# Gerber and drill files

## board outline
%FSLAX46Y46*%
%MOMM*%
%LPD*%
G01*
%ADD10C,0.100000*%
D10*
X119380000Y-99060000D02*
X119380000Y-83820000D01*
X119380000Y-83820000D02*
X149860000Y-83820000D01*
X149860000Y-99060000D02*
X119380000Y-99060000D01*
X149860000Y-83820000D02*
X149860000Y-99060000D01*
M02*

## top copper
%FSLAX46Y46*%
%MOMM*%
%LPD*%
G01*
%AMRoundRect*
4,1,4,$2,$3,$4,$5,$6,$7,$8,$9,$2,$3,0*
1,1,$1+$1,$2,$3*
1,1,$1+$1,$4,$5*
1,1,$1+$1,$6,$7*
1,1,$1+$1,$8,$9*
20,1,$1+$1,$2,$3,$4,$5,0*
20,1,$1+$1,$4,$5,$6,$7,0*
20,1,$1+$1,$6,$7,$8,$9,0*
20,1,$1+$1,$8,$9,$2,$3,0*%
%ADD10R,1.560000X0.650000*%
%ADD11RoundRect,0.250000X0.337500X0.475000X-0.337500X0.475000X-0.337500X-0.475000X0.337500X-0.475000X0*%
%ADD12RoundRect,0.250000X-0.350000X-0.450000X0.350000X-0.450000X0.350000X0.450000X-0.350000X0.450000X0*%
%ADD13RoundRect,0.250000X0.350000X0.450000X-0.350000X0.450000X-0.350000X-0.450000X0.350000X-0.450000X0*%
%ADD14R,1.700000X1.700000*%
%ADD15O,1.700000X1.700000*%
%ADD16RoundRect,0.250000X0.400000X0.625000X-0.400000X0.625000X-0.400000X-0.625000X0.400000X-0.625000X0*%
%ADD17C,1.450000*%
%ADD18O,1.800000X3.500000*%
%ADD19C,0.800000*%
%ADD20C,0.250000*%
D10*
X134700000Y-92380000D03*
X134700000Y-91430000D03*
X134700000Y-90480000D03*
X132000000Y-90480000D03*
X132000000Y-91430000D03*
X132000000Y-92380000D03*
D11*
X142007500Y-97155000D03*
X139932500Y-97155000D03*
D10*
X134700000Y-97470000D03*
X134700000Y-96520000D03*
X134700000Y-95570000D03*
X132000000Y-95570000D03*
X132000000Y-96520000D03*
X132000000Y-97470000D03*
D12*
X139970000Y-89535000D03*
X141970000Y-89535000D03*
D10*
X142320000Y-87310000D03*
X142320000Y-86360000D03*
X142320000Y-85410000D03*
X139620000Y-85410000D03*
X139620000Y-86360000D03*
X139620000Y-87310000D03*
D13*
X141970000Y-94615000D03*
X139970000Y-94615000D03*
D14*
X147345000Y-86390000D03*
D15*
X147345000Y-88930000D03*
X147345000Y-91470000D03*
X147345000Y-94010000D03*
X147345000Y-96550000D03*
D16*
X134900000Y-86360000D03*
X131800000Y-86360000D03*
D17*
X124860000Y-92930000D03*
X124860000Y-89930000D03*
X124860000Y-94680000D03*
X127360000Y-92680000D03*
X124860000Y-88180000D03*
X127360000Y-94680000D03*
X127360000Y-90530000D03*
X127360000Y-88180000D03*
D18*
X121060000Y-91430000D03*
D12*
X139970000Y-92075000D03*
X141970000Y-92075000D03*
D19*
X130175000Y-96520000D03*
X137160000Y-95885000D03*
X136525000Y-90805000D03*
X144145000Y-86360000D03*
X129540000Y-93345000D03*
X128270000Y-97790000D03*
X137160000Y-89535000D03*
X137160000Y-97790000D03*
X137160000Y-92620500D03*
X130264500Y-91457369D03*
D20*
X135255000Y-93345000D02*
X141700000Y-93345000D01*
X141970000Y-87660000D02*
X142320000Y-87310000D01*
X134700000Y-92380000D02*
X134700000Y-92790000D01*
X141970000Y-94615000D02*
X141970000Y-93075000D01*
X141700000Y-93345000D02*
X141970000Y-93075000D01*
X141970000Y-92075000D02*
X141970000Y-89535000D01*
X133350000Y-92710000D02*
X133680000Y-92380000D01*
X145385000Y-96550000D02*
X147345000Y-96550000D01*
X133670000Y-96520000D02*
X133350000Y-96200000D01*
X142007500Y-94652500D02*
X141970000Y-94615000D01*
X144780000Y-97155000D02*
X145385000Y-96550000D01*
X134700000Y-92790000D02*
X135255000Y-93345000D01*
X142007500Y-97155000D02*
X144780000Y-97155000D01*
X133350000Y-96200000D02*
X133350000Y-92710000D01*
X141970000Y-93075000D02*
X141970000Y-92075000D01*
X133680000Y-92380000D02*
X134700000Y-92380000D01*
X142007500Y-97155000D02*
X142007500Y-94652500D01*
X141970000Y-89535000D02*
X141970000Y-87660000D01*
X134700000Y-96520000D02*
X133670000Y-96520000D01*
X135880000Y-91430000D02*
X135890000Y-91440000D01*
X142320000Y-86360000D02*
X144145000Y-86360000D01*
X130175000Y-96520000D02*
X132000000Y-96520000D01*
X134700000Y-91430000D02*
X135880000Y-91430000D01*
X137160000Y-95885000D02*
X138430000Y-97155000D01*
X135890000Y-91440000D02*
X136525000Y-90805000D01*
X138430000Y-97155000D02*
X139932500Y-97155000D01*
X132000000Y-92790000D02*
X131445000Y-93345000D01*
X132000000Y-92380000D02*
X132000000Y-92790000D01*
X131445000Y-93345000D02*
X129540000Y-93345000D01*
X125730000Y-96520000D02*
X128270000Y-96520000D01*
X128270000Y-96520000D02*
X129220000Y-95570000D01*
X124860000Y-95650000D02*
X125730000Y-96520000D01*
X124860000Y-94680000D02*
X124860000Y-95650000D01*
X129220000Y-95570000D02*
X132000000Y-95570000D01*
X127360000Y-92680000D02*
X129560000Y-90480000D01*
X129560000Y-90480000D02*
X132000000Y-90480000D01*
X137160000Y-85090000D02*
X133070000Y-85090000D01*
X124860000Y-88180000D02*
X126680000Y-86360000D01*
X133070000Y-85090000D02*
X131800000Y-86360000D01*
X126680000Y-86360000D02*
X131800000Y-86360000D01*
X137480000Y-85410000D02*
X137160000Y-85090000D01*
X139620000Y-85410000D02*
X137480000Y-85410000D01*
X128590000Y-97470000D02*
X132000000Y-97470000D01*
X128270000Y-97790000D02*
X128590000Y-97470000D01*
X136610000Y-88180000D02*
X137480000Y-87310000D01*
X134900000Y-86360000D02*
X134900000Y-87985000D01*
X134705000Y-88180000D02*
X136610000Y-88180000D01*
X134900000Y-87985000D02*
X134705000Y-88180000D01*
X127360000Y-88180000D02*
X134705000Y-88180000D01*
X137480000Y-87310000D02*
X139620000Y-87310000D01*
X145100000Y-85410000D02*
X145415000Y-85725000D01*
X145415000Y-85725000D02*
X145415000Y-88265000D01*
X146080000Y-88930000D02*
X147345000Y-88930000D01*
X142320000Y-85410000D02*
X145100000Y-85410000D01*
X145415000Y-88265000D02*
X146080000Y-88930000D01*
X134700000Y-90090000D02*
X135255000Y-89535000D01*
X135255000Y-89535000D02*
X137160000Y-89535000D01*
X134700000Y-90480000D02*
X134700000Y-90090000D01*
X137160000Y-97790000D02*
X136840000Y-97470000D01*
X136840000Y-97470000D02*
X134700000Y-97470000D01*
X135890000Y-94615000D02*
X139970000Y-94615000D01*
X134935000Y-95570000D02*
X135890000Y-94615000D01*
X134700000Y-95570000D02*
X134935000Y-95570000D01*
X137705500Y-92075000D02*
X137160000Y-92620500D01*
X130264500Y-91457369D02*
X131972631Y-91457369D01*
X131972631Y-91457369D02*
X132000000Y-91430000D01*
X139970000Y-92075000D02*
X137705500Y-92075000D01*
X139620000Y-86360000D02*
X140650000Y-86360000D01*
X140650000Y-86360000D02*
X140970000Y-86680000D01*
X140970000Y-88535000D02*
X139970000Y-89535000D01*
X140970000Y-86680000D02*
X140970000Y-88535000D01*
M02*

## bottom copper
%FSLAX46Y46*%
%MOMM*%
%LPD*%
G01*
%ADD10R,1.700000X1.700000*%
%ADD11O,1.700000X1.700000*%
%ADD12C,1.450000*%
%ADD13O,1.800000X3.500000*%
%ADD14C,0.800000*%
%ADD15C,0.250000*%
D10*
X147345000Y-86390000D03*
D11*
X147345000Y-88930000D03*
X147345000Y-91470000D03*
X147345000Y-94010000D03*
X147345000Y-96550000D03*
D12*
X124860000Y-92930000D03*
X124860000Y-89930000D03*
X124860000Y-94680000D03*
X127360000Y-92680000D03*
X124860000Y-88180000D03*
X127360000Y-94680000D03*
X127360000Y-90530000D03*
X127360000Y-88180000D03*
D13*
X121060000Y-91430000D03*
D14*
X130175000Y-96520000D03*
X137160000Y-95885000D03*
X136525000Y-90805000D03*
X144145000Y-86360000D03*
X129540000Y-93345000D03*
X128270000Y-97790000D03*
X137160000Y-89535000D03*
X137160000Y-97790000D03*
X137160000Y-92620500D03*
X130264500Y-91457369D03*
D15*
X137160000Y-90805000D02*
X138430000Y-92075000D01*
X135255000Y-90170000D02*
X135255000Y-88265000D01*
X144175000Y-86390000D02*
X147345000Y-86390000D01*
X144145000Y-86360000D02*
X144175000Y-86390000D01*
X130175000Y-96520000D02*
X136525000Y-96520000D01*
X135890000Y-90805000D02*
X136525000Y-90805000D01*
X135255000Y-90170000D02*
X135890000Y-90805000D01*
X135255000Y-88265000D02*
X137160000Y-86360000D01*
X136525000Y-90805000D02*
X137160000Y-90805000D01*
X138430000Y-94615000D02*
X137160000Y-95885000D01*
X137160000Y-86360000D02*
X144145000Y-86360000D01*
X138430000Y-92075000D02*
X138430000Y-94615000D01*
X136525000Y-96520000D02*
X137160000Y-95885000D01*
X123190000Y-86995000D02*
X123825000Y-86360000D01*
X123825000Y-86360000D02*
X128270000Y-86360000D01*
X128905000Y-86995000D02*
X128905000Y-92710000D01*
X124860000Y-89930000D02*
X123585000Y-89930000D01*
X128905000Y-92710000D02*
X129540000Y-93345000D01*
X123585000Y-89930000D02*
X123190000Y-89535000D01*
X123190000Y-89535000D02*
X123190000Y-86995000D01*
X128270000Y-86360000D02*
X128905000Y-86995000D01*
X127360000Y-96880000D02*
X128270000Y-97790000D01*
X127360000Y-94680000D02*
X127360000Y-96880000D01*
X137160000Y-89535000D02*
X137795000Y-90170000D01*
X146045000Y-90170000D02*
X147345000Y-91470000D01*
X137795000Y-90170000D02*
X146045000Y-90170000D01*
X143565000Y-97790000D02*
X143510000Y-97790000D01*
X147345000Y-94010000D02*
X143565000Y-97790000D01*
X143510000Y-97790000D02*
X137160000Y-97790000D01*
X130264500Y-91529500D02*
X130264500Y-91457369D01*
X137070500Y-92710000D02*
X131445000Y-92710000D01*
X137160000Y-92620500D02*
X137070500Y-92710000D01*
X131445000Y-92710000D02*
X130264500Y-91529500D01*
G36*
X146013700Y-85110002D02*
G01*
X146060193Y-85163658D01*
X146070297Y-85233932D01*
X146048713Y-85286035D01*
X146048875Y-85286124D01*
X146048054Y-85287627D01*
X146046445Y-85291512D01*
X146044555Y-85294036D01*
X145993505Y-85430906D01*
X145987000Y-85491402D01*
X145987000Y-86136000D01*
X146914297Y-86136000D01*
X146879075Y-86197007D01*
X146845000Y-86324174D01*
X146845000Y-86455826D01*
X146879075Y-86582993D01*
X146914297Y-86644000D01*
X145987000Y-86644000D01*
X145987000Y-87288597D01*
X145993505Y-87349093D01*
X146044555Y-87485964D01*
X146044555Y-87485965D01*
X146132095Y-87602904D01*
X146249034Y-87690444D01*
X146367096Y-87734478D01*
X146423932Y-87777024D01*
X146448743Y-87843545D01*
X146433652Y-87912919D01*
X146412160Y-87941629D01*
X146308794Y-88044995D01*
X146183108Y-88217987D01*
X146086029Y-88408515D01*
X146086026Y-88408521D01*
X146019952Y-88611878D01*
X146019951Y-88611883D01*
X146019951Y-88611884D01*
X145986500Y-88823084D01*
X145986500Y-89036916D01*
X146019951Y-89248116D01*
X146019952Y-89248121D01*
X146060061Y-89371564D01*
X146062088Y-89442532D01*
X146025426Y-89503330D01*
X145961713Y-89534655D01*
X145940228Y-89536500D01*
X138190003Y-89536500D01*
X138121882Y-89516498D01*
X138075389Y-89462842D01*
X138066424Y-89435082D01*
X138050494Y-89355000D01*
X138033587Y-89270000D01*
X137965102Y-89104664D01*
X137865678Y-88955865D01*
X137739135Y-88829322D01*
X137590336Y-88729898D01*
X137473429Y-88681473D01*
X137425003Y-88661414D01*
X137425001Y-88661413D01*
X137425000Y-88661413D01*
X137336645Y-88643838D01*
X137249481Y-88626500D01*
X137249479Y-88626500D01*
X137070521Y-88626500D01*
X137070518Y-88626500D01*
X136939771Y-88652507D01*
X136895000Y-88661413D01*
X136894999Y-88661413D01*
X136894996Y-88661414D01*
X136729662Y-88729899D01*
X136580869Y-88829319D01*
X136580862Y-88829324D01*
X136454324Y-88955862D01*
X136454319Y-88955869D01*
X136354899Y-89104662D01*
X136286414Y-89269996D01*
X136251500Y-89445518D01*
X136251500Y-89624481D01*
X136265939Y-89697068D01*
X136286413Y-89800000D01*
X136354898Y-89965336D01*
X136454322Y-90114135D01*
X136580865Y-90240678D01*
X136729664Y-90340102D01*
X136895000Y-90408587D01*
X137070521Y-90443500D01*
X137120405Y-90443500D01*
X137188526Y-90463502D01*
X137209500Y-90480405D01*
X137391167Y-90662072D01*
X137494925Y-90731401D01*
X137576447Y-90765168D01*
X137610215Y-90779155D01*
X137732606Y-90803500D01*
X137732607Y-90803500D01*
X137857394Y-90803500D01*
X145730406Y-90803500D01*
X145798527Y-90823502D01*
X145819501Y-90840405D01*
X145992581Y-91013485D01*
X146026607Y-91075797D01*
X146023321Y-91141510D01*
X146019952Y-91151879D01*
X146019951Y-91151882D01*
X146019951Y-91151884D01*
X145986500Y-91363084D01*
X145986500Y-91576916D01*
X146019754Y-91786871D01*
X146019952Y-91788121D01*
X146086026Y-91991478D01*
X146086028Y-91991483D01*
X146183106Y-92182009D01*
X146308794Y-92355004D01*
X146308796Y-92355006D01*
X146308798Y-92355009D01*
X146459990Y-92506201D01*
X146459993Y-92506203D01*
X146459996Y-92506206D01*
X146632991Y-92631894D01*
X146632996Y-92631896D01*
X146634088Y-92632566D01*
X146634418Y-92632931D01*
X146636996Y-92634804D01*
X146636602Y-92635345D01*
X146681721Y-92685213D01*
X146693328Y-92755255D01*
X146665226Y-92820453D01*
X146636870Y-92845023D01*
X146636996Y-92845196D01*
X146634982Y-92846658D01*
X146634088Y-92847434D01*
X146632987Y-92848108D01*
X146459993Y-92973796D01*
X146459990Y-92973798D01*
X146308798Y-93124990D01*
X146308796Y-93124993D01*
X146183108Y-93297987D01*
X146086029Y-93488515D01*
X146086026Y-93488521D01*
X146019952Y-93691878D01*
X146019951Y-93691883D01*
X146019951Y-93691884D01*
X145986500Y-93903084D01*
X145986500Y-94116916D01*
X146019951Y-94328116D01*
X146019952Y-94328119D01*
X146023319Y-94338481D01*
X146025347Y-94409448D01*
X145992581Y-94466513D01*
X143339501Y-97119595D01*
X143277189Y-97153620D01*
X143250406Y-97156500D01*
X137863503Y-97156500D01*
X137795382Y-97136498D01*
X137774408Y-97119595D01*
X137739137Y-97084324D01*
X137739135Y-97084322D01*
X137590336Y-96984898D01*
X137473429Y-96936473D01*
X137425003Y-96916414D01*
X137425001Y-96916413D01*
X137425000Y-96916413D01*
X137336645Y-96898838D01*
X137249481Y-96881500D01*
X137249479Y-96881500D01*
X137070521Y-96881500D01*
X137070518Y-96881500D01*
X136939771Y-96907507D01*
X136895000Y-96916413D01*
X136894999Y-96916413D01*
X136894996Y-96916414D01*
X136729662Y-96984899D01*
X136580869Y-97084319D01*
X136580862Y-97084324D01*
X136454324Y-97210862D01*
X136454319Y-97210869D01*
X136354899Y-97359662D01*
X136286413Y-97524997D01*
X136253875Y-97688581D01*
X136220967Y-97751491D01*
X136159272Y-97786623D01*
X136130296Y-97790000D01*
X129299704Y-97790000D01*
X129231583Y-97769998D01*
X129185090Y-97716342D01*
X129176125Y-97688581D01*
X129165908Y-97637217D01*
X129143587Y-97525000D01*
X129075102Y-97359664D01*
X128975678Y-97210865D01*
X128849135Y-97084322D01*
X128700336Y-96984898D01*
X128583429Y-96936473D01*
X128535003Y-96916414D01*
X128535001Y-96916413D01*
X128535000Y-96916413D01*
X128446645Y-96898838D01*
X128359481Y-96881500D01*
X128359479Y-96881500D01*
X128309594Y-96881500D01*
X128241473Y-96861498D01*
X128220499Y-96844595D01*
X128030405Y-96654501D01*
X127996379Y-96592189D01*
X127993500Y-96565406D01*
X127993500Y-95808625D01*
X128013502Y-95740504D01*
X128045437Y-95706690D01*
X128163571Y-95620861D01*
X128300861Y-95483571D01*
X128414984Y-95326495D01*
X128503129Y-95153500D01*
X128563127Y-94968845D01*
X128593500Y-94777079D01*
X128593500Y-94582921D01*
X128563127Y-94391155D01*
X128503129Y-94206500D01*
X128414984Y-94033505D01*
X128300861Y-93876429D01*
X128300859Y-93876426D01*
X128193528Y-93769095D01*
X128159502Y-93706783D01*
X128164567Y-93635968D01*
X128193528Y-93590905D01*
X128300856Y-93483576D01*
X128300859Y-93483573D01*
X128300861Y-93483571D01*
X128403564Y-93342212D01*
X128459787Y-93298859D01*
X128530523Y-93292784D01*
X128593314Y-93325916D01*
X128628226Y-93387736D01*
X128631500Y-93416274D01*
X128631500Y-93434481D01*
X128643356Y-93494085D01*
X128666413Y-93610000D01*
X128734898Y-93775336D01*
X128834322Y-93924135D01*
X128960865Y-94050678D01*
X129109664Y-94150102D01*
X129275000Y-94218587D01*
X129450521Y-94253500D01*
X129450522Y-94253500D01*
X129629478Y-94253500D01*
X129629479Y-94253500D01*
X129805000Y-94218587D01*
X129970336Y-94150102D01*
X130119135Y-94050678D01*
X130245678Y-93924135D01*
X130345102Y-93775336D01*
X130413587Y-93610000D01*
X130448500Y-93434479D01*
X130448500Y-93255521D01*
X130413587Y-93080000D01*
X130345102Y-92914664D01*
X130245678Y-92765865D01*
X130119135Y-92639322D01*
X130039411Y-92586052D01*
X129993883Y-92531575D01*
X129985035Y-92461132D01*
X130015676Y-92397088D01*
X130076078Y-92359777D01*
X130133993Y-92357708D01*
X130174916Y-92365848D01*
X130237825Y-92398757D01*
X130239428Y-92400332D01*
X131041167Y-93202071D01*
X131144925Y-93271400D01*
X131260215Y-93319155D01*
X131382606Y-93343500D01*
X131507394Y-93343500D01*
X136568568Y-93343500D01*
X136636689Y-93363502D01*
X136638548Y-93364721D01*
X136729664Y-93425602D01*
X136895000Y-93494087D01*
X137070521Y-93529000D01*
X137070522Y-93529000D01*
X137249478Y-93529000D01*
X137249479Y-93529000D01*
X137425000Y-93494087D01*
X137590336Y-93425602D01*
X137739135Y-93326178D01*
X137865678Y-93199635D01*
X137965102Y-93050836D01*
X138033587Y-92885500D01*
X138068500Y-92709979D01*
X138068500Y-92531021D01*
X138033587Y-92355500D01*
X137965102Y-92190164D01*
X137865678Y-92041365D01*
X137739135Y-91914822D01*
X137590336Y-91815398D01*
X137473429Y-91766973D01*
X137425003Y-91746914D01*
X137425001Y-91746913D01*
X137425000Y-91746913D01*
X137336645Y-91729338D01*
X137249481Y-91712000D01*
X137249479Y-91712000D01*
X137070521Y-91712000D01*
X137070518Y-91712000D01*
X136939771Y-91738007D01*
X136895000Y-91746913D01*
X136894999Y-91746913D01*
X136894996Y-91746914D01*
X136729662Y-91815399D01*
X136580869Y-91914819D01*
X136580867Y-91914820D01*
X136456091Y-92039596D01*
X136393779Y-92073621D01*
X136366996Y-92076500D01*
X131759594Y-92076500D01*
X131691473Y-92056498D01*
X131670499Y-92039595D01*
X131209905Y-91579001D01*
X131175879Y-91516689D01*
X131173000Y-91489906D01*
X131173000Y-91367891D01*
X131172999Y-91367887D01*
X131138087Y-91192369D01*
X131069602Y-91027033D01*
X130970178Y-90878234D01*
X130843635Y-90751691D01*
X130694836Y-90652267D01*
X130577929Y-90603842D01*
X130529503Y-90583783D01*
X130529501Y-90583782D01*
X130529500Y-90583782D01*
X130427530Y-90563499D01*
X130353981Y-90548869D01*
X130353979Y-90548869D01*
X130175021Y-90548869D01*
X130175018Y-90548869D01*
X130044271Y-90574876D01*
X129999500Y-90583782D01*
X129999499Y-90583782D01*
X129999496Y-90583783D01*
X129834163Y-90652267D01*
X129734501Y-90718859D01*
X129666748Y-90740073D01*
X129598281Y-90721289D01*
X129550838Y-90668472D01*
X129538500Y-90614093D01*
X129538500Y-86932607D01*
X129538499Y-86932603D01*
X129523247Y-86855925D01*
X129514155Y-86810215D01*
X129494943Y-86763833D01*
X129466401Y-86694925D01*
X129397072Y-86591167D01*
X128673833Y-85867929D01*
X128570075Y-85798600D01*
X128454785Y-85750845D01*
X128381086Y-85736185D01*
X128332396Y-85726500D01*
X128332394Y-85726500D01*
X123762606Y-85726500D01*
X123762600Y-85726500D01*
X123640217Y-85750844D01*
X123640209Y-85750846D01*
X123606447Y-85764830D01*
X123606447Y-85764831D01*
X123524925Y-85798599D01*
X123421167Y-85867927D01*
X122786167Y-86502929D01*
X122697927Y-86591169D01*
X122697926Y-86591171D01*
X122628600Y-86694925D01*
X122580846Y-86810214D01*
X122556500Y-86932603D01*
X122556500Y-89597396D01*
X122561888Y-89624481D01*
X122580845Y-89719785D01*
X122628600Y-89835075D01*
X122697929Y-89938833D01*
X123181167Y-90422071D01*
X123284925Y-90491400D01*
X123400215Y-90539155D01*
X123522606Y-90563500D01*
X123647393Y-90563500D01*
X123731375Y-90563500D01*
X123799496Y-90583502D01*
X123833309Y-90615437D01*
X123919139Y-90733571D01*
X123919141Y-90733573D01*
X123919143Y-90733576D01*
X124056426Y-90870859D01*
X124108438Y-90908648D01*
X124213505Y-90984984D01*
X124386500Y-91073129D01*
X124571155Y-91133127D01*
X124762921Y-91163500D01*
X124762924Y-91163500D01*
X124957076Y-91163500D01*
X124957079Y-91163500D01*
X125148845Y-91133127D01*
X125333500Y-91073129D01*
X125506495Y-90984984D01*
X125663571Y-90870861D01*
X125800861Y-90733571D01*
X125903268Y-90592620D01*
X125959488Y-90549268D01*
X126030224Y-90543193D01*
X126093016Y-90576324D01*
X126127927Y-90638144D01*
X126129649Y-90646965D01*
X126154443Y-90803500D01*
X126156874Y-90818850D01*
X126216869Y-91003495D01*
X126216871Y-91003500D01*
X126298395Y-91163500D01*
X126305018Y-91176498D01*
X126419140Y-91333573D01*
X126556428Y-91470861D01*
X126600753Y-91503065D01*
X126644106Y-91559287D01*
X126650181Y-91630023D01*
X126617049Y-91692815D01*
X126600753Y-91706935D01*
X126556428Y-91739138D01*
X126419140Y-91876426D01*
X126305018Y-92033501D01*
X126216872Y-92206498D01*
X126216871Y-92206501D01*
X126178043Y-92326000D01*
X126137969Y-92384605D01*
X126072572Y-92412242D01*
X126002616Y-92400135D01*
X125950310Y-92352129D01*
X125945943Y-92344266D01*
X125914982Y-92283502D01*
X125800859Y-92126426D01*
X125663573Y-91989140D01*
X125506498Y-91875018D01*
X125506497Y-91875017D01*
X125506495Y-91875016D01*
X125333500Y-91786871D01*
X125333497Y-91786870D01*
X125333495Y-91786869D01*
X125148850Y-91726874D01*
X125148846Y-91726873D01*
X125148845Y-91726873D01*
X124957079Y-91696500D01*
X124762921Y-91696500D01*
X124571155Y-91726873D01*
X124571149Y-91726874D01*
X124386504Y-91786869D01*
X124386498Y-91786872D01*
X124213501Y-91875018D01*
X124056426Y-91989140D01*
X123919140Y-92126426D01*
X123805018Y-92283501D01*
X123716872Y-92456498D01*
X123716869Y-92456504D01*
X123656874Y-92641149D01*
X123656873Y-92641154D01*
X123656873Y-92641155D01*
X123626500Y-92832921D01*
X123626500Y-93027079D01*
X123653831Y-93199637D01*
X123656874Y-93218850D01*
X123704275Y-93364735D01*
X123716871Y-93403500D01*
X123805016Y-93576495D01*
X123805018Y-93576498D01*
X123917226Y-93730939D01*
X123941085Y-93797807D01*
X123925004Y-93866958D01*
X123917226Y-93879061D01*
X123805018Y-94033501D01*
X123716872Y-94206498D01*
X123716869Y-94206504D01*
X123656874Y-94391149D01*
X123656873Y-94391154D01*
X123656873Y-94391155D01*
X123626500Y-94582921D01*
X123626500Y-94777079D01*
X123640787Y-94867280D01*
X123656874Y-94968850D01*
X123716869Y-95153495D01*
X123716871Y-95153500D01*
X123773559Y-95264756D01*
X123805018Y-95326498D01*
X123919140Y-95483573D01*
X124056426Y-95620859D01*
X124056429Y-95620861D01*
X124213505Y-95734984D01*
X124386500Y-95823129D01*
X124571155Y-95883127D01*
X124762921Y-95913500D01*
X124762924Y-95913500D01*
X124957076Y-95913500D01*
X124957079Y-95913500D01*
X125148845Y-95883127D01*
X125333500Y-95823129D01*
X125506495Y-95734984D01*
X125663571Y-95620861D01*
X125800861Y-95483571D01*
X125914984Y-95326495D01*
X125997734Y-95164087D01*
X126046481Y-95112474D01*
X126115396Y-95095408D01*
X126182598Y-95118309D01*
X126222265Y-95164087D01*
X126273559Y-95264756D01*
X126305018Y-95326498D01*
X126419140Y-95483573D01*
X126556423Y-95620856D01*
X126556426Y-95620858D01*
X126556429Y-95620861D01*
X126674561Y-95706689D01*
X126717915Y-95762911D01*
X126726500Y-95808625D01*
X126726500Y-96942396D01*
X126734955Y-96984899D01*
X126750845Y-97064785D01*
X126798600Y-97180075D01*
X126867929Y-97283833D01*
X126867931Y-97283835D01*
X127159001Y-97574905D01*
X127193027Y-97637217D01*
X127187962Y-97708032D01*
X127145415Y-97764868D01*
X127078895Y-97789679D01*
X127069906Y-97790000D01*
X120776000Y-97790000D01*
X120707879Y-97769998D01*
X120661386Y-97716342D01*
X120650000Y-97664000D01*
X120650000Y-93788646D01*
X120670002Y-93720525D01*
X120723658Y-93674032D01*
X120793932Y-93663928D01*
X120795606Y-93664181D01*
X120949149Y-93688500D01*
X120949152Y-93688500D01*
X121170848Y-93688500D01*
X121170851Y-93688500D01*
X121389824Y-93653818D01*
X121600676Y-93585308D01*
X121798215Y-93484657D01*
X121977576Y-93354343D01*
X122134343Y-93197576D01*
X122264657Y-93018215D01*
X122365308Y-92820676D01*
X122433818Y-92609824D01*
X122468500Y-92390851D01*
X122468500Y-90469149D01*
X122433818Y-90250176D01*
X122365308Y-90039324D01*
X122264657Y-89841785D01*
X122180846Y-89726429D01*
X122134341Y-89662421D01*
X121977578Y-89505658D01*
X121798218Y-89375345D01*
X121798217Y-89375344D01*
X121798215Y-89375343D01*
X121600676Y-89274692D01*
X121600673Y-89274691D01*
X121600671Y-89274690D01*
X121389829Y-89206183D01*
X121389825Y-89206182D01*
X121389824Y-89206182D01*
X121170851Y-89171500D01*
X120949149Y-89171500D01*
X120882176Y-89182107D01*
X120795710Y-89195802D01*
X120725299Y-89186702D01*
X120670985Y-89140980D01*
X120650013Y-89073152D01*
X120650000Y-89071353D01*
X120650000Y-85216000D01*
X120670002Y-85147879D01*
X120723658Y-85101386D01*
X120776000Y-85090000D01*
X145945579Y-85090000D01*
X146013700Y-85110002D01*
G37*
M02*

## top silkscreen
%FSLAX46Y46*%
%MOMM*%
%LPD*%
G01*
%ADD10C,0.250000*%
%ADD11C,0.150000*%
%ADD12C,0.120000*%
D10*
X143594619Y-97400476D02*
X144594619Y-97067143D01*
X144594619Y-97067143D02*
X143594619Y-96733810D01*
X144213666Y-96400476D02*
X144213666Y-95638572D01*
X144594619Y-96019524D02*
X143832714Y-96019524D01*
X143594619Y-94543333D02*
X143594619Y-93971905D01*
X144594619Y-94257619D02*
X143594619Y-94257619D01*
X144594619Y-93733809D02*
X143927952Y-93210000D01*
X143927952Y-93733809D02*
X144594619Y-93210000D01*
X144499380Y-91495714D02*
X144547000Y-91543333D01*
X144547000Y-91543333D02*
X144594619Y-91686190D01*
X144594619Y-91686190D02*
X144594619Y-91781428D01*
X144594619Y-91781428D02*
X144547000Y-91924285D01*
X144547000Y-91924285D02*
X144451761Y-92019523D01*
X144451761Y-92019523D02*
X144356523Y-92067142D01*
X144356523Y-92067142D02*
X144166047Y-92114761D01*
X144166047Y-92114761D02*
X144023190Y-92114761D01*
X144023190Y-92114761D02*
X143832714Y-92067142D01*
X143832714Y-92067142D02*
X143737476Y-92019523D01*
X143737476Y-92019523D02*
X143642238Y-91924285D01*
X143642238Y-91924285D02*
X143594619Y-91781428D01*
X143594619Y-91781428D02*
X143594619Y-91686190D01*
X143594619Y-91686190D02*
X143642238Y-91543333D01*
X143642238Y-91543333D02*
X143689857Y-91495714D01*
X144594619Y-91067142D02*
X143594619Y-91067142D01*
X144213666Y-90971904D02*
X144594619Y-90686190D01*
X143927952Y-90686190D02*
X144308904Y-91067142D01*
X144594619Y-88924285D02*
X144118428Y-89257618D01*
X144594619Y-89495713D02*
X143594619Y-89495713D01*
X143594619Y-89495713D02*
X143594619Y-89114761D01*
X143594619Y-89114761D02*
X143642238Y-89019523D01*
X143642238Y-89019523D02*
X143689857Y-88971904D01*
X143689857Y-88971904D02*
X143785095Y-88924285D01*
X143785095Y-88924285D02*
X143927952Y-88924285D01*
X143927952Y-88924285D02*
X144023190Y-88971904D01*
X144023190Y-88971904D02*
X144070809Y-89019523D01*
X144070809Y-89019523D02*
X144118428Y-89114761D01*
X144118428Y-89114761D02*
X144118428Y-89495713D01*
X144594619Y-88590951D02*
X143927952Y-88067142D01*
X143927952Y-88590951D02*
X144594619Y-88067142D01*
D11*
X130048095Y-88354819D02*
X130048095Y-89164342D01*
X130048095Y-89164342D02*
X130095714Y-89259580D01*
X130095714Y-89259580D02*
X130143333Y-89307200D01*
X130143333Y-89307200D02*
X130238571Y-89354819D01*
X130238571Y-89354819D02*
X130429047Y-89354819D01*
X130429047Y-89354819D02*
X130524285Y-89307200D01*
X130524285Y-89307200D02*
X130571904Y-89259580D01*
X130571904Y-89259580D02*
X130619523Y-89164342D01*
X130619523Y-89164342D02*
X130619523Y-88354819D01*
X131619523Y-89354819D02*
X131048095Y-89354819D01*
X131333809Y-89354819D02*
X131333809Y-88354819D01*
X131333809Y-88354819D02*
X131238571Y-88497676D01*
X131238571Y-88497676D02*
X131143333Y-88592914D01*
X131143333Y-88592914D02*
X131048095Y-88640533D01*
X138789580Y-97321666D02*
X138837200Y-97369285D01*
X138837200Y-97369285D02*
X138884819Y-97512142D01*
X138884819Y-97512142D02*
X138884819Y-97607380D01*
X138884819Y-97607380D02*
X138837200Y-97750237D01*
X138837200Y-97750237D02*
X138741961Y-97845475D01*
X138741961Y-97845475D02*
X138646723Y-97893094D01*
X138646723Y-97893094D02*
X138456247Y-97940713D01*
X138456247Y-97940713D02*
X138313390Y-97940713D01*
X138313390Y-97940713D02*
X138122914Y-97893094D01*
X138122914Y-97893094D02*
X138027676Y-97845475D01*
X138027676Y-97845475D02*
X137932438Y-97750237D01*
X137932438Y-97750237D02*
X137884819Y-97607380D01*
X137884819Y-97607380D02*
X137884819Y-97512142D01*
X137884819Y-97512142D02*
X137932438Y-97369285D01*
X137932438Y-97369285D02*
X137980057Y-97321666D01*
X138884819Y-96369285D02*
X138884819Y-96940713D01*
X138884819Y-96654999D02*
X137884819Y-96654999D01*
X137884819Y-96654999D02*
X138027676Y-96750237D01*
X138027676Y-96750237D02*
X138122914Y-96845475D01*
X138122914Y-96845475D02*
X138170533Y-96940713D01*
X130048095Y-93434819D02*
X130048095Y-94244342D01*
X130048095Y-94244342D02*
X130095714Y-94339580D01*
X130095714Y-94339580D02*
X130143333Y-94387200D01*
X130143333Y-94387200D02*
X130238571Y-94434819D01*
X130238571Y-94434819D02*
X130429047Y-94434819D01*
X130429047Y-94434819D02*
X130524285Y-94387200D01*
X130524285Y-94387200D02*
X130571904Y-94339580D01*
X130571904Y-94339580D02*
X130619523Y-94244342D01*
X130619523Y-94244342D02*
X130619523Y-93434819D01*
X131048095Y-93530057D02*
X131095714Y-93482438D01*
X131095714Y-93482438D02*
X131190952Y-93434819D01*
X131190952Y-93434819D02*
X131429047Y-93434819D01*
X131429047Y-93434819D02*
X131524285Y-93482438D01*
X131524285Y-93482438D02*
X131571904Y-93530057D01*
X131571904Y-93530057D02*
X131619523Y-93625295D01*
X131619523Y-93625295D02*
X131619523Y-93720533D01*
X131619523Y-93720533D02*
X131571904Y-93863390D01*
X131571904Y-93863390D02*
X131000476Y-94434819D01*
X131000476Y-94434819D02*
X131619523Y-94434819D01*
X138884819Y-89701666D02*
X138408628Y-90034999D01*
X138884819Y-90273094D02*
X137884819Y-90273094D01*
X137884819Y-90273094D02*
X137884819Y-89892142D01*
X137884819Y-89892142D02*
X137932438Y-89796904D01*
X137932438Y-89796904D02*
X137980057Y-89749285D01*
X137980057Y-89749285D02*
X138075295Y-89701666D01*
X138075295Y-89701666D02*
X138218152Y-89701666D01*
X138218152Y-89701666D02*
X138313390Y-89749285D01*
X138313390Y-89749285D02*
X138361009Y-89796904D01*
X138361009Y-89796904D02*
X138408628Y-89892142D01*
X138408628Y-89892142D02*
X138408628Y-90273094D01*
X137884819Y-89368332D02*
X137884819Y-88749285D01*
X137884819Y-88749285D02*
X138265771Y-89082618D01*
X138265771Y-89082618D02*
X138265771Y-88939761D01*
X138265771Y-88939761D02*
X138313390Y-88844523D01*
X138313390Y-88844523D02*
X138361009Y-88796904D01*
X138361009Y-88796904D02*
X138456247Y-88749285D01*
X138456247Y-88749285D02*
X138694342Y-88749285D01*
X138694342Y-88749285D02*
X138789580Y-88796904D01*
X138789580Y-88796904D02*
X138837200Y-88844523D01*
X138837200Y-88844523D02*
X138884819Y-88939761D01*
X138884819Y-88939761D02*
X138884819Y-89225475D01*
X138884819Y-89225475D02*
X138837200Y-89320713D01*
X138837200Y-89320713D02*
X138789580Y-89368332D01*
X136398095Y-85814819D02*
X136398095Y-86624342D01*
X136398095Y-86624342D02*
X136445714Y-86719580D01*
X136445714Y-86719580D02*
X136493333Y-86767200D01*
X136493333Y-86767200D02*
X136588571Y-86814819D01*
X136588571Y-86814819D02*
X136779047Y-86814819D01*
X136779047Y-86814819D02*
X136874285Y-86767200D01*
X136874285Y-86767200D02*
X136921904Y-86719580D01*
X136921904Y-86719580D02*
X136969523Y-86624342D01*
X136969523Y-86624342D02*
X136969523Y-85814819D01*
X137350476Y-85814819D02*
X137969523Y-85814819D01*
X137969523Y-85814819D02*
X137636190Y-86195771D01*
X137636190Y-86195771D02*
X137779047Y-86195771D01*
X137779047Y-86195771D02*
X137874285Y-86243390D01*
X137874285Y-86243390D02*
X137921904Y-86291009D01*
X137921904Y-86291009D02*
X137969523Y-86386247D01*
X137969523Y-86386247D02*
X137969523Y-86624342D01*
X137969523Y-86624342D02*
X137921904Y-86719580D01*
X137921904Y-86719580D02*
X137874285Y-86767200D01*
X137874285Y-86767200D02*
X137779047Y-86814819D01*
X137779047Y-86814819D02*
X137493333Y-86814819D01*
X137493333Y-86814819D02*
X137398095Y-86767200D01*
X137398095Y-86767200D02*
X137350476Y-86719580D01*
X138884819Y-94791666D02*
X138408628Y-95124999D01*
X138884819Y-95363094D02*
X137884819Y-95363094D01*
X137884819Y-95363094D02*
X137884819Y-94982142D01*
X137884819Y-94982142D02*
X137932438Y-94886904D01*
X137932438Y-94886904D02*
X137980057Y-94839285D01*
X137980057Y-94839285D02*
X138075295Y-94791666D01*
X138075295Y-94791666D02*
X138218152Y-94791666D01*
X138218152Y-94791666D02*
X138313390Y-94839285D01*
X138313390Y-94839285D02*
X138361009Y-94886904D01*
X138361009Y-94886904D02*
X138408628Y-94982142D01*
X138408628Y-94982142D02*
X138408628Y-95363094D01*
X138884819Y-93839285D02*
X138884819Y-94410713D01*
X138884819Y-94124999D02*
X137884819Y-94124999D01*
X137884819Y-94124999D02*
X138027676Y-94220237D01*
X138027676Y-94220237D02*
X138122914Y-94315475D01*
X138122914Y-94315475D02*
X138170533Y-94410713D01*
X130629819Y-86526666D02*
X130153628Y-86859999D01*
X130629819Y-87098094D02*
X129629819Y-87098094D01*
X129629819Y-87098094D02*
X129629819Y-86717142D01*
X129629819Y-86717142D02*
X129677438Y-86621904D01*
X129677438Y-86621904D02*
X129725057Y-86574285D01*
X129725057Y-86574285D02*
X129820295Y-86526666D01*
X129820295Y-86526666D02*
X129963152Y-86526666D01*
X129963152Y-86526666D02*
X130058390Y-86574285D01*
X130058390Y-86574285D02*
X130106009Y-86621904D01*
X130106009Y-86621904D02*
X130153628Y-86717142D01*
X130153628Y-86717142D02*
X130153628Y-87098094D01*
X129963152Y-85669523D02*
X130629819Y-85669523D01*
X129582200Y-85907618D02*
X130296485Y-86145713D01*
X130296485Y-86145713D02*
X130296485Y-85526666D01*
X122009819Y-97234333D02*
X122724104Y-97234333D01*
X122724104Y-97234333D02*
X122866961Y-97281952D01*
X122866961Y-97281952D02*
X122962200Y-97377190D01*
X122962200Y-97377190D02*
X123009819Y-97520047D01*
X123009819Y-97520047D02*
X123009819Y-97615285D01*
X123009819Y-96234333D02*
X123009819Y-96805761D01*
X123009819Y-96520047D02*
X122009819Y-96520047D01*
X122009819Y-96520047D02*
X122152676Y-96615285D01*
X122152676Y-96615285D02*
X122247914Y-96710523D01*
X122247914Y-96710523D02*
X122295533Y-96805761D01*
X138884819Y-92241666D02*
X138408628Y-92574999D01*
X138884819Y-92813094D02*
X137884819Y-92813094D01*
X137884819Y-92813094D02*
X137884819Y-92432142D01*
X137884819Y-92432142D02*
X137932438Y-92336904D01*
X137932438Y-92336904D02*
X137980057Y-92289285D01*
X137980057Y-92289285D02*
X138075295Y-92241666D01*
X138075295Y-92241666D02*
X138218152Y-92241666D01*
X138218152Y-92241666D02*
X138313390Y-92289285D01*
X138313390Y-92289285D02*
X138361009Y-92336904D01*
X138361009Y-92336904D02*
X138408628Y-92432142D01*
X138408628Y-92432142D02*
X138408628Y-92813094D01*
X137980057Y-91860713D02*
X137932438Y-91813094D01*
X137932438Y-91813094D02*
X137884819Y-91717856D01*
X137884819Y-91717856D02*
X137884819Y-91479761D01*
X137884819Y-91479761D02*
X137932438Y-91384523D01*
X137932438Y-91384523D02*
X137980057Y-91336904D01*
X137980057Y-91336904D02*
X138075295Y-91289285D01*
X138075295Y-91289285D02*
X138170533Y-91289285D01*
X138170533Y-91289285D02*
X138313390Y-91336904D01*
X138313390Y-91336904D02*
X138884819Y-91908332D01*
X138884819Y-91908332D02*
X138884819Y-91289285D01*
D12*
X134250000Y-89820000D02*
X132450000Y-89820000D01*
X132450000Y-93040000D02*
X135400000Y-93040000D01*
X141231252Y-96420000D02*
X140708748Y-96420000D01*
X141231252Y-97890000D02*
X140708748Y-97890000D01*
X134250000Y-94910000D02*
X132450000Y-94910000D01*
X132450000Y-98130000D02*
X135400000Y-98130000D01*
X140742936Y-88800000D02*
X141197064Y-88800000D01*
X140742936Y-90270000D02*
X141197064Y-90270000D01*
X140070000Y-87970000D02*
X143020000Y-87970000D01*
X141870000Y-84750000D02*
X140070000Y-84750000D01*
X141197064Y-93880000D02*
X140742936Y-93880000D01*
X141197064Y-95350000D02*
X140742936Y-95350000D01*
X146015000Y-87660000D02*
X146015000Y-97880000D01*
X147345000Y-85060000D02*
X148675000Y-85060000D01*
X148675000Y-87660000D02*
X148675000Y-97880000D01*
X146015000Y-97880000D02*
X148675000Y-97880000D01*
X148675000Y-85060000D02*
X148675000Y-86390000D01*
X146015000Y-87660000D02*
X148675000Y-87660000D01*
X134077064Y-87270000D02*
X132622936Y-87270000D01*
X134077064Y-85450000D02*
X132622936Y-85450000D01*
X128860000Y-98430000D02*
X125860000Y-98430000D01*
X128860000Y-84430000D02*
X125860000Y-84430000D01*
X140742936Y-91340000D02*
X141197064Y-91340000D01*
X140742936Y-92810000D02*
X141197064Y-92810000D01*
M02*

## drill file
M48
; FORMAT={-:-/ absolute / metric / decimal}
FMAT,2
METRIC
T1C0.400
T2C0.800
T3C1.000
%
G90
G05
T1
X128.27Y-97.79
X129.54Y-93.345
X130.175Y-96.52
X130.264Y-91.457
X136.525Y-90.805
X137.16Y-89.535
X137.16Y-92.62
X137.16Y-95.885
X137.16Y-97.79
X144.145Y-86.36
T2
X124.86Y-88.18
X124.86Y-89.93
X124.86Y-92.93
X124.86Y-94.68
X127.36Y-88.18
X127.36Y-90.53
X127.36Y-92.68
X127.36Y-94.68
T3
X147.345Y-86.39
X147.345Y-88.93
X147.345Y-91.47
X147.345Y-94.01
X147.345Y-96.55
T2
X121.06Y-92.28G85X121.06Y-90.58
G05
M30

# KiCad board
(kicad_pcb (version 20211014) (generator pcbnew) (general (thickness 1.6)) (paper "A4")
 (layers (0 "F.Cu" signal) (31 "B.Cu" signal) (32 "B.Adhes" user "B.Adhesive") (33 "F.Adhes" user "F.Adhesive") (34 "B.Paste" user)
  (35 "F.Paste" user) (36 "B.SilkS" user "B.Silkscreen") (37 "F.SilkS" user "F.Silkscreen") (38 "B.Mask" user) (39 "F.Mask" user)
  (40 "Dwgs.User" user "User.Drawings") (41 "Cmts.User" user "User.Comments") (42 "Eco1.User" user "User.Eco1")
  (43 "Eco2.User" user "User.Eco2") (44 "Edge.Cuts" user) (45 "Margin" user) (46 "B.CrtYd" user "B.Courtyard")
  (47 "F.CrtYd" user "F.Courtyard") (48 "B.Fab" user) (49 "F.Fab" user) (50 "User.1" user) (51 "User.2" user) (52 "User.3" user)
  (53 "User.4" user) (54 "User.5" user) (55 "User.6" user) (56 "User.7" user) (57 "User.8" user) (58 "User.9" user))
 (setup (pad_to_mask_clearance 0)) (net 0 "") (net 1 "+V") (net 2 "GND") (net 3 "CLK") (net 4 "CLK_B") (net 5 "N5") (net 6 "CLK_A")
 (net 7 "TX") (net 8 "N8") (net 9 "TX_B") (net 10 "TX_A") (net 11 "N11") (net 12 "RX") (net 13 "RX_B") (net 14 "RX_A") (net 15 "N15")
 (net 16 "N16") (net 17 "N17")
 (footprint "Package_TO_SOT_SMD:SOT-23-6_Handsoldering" (layer "F.Cu") (at 133.35 91.43 180)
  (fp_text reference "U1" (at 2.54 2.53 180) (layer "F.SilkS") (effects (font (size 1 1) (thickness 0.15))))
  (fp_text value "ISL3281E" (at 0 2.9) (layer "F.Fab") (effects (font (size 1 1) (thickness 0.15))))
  (fp_line (start -0.9 1.61) (end 0.9 1.61) (layer "F.SilkS") (width 0.12))
  (fp_line (start 0.9 -1.61) (end -2.05 -1.61) (layer "F.SilkS") (width 0.12))
  (pad "1" smd rect (at -1.35 -0.95 180) (size 1.56 0.65) (layers "F.Cu" "F.Paste" "F.Mask") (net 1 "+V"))
  (pad "2" smd rect (at -1.35 0 180) (size 1.56 0.65) (layers "F.Cu" "F.Paste" "F.Mask") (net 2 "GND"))
  (pad "3" smd rect (at -1.35 0.95 180) (size 1.56 0.65) (layers "F.Cu" "F.Paste" "F.Mask") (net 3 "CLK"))
  (pad "4" smd rect (at 1.35 0.95 180) (size 1.56 0.65) (layers "F.Cu" "F.Paste" "F.Mask") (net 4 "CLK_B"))
  (pad "5" smd rect (at 1.35 0 180) (size 1.56 0.65) (layers "F.Cu" "F.Paste" "F.Mask") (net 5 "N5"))
  (pad "6" smd rect (at 1.35 -0.95 180) (size 1.56 0.65) (layers "F.Cu" "F.Paste" "F.Mask") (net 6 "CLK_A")))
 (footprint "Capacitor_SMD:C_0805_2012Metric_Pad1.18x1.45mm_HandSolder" (layer "F.Cu") (at 140.97 97.155 180)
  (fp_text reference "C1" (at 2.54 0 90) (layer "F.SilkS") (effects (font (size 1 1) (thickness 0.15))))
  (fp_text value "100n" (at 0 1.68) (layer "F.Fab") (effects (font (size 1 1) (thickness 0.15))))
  (fp_line (start -0.261252 0.735) (end 0.261252 0.735) (layer "F.SilkS") (width 0.12))
  (fp_line (start -0.261252 -0.735) (end 0.261252 -0.735) (layer "F.SilkS") (width 0.12))
  (pad "1" smd roundrect (at -1.0375 0 180) (size 1.175 1.45) (layers "F.Cu" "F.Paste" "F.Mask") (roundrect_rratio 0.2127659574)
   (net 1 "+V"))
  (pad "2" smd roundrect (at 1.0375 0 180) (size 1.175 1.45) (layers "F.Cu" "F.Paste" "F.Mask") (roundrect_rratio 0.2127659574)
   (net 2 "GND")))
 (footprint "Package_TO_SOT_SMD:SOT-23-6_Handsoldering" (layer "F.Cu") (at 133.35 96.52 180)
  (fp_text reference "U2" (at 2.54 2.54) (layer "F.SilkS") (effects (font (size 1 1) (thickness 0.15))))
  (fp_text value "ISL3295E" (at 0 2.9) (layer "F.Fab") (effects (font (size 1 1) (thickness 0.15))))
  (fp_line (start -0.9 1.61) (end 0.9 1.61) (layer "F.SilkS") (width 0.12))
  (fp_line (start 0.9 -1.61) (end -2.05 -1.61) (layer "F.SilkS") (width 0.12))
  (pad "1" smd rect (at -1.35 -0.95 180) (size 1.56 0.65) (layers "F.Cu" "F.Paste" "F.Mask") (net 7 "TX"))
  (pad "2" smd rect (at -1.35 0 180) (size 1.56 0.65) (layers "F.Cu" "F.Paste" "F.Mask") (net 1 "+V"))
  (pad "3" smd rect (at -1.35 0.95 180) (size 1.56 0.65) (layers "F.Cu" "F.Paste" "F.Mask") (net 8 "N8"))
  (pad "4" smd rect (at 1.35 0.95 180) (size 1.56 0.65) (layers "F.Cu" "F.Paste" "F.Mask") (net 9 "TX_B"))
  (pad "5" smd rect (at 1.35 0 180) (size 1.56 0.65) (layers "F.Cu" "F.Paste" "F.Mask") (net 2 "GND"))
  (pad "6" smd rect (at 1.35 -0.95 180) (size 1.56 0.65) (layers "F.Cu" "F.Paste" "F.Mask") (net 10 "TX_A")))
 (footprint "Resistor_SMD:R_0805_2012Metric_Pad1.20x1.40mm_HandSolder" (layer "F.Cu") (at 140.97 89.535)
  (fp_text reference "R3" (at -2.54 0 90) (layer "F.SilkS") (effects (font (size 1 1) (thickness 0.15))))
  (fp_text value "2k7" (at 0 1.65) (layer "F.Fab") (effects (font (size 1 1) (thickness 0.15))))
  (fp_line (start -0.227064 -0.735) (end 0.227064 -0.735) (layer "F.SilkS") (width 0.12))
  (fp_line (start -0.227064 0.735) (end 0.227064 0.735) (layer "F.SilkS") (width 0.12))
  (pad "1" smd roundrect (at -1 0) (size 1.2 1.4) (layers "F.Cu" "F.Paste" "F.Mask") (roundrect_rratio 0.2083333333) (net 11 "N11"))
  (pad "2" smd roundrect (at 1 0) (size 1.2 1.4) (layers "F.Cu" "F.Paste" "F.Mask") (roundrect_rratio 0.2083333333) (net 1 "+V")))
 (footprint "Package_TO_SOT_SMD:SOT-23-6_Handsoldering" (layer "F.Cu") (at 140.97 86.36 180)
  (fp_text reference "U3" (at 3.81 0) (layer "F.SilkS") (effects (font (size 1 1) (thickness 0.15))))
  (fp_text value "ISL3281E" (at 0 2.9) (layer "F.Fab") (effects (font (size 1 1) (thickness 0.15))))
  (fp_line (start 0.9 -1.61) (end -2.05 -1.61) (layer "F.SilkS") (width 0.12))
  (fp_line (start -0.9 1.61) (end 0.9 1.61) (layer "F.SilkS") (width 0.12))
  (pad "1" smd rect (at -1.35 -0.95 180) (size 1.56 0.65) (layers "F.Cu" "F.Paste" "F.Mask") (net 1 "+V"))
  (pad "2" smd rect (at -1.35 0 180) (size 1.56 0.65) (layers "F.Cu" "F.Paste" "F.Mask") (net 2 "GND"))
  (pad "3" smd rect (at -1.35 0.95 180) (size 1.56 0.65) (layers "F.Cu" "F.Paste" "F.Mask") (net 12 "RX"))
  (pad "4" smd rect (at 1.35 0.95 180) (size 1.56 0.65) (layers "F.Cu" "F.Paste" "F.Mask") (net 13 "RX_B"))
  (pad "5" smd rect (at 1.35 0 180) (size 1.56 0.65) (layers "F.Cu" "F.Paste" "F.Mask") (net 11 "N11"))
  (pad "6" smd rect (at 1.35 -0.95 180) (size 1.56 0.65) (layers "F.Cu" "F.Paste" "F.Mask") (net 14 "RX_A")))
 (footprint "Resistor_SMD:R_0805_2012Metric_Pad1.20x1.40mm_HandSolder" (layer "F.Cu") (at 140.97 94.615 180)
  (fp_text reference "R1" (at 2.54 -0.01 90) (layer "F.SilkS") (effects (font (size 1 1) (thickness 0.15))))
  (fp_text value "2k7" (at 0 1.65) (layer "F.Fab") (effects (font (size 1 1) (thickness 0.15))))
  (fp_line (start -0.227064 0.735) (end 0.227064 0.735) (layer "F.SilkS") (width 0.12))
  (fp_line (start -0.227064 -0.735) (end 0.227064 -0.735) (layer "F.SilkS") (width 0.12))
  (pad "1" smd roundrect (at -1 0 180) (size 1.2 1.4) (layers "F.Cu" "F.Paste" "F.Mask") (roundrect_rratio 0.2083333333) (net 1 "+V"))
  (pad "2" smd roundrect (at 1 0 180) (size 1.2 1.4) (layers "F.Cu" "F.Paste" "F.Mask") (roundrect_rratio 0.2083333333) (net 8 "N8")))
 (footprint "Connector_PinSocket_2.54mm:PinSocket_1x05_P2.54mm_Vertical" (layer "F.Cu") (at 147.345 86.39)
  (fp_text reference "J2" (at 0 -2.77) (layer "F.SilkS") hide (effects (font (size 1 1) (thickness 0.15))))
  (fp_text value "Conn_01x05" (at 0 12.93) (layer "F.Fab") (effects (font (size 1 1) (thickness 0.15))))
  (fp_line (start -1.33 1.27) (end -1.33 11.49) (layer "F.SilkS") (width 0.12))
  (fp_line (start 0 -1.33) (end 1.33 -1.33) (layer "F.SilkS") (width 0.12))
  (fp_line (start 1.33 1.27) (end 1.33 11.49) (layer "F.SilkS") (width 0.12))
  (fp_line (start -1.33 11.49) (end 1.33 11.49) (layer "F.SilkS") (width 0.12))
  (fp_line (start 1.33 -1.33) (end 1.33 0) (layer "F.SilkS") (width 0.12))
  (fp_line (start -1.33 1.27) (end 1.33 1.27) (layer "F.SilkS") (width 0.12))
  (pad "1" thru_hole rect (at 0 0) (size 1.7 1.7) (drill 1) (layers *.Cu *.Mask) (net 2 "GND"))
  (pad "2" thru_hole oval (at 0 2.54) (size 1.7 1.7) (drill 1) (layers *.Cu *.Mask) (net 12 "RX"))
  (pad "3" thru_hole oval (at 0 5.08) (size 1.7 1.7) (drill 1) (layers *.Cu *.Mask) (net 3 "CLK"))
  (pad "4" thru_hole oval (at 0 7.62) (size 1.7 1.7) (drill 1) (layers *.Cu *.Mask) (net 7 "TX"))
  (pad "5" thru_hole oval (at 0 10.16) (size 1.7 1.7) (drill 1) (layers *.Cu *.Mask) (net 1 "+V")))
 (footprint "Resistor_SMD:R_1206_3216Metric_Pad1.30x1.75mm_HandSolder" (layer "F.Cu") (at 133.35 86.36 180)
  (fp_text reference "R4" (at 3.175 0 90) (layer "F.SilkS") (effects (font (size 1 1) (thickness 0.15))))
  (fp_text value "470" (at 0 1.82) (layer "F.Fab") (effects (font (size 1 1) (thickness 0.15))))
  (fp_line (start -0.727064 -0.91) (end 0.727064 -0.91) (layer "F.SilkS") (width 0.12))
  (fp_line (start -0.727064 0.91) (end 0.727064 0.91) (layer "F.SilkS") (width 0.12))
  (pad "1" smd roundrect (at -1.55 0 180) (size 1.3 1.75) (layers "F.Cu" "F.Paste" "F.Mask") (roundrect_rratio 0.1923076923) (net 14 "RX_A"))
  (pad "2" smd roundrect (at 1.55 0 180) (size 1.3 1.75) (layers "F.Cu" "F.Paste" "F.Mask") (roundrect_rratio 0.1923076923) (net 13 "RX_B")))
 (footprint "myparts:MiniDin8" (layer "F.Cu") (at 116.36 91.43 90)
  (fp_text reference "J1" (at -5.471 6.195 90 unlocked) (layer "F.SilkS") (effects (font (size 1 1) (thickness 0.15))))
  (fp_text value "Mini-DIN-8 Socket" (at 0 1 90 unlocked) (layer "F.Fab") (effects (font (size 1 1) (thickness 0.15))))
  (fp_line (start -7 12.5) (end -7 9.5) (layer "F.SilkS") (width 0.12))
  (fp_line (start 7 12.5) (end 7 9.5) (layer "F.SilkS") (width 0.12))
  (pad "1" thru_hole circle (at -1.5 8.5 90) (size 1.45 1.45) (drill 0.8) (layers *.Cu *.Mask) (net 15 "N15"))
  (pad "2" thru_hole circle (at 1.5 8.5 90) (size 1.45 1.45) (drill 0.8) (layers *.Cu *.Mask) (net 6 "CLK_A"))
  (pad "3" thru_hole circle (at -3.25 8.5 90) (size 1.45 1.45) (drill 0.8) (layers *.Cu *.Mask) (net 9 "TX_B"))
  (pad "4" thru_hole circle (at -1.25 11 90) (size 1.45 1.45) (drill 0.8) (layers *.Cu *.Mask) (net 4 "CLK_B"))
  (pad "5" thru_hole circle (at 3.25 8.5 90) (size 1.45 1.45) (drill 0.8) (layers *.Cu *.Mask) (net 13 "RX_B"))
  (pad "6" thru_hole circle (at -3.25 11 90) (size 1.45 1.45) (drill 0.8) (layers *.Cu *.Mask) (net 10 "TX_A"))
  (pad "7" thru_hole circle (at 0.9 11 90) (size 1.45 1.45) (drill 0.8) (layers *.Cu *.Mask) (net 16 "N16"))
  (pad "8" thru_hole circle (at 3.25 11 90) (size 1.45 1.45) (drill 0.8) (layers *.Cu *.Mask) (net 14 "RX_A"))
  (pad "9" thru_hole oval (at 0 4.7 90) (size 3.5 1.8) (drill oval 2.5 0.8) (layers *.Cu *.Mask) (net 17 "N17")))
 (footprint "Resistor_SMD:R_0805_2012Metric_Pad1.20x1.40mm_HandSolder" (layer "F.Cu") (at 140.97 92.075)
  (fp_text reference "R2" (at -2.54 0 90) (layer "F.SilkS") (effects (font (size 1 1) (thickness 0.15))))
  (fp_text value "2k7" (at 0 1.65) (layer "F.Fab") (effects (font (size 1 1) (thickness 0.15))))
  (fp_line (start -0.227064 -0.735) (end 0.227064 -0.735) (layer "F.SilkS") (width 0.12))
  (fp_line (start -0.227064 0.735) (end 0.227064 0.735) (layer "F.SilkS") (width 0.12))
  (pad "1" smd roundrect (at -1 0) (size 1.2 1.4) (layers "F.Cu" "F.Paste" "F.Mask") (roundrect_rratio 0.2083333333) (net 5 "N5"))
  (pad "2" smd roundrect (at 1 0) (size 1.2 1.4) (layers "F.Cu" "F.Paste" "F.Mask") (roundrect_rratio 0.2083333333) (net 1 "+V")))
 (gr_line (start 119.38 99.06) (end 119.38 83.82) (layer "Edge.Cuts") (width 0.1))
 (gr_line (start 119.38 83.82) (end 149.86 83.82) (layer "Edge.Cuts") (width 0.1))
 (gr_line (start 149.86 99.06) (end 119.38 99.06) (layer "Edge.Cuts") (width 0.1))
 (gr_line (start 149.86 83.82) (end 149.86 99.06) (layer "Edge.Cuts") (width 0.1))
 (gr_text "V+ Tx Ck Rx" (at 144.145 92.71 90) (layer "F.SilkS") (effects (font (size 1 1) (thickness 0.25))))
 (segment (start 135.255 93.345) (end 141.7 93.345) (width 0.25) (layer "F.Cu") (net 1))
 (segment (start 141.97 87.66) (end 142.32 87.31) (width 0.25) (layer "F.Cu") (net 1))
 (segment (start 134.7 92.38) (end 134.7 92.79) (width 0.25) (layer "F.Cu") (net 1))
 (segment (start 141.97 94.615) (end 141.97 93.075) (width 0.25) (layer "F.Cu") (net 1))
 (segment (start 141.7 93.345) (end 141.97 93.075) (width 0.25) (layer "F.Cu") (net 1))
 (segment (start 141.97 92.075) (end 141.97 89.535) (width 0.25) (layer "F.Cu") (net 1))
 (segment (start 133.35 92.71) (end 133.68 92.38) (width 0.25) (layer "F.Cu") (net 1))
 (segment (start 145.385 96.55) (end 147.345 96.55) (width 0.25) (layer "F.Cu") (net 1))
 (segment (start 133.67 96.52) (end 133.35 96.2) (width 0.25) (layer "F.Cu") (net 1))
 (segment (start 142.0075 94.6525) (end 141.97 94.615) (width 0.25) (layer "F.Cu") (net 1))
 (segment (start 144.78 97.155) (end 145.385 96.55) (width 0.25) (layer "F.Cu") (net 1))
 (segment (start 134.7 92.79) (end 135.255 93.345) (width 0.25) (layer "F.Cu") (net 1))
 (segment (start 142.0075 97.155) (end 144.78 97.155) (width 0.25) (layer "F.Cu") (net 1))
 (segment (start 133.35 96.2) (end 133.35 92.71) (width 0.25) (layer "F.Cu") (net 1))
 (segment (start 141.97 93.075) (end 141.97 92.075) (width 0.25) (layer "F.Cu") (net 1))
 (segment (start 133.68 92.38) (end 134.7 92.38) (width 0.25) (layer "F.Cu") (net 1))
 (segment (start 142.0075 97.155) (end 142.0075 94.6525) (width 0.25) (layer "F.Cu") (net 1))
 (segment (start 141.97 89.535) (end 141.97 87.66) (width 0.25) (layer "F.Cu") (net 1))
 (segment (start 134.7 96.52) (end 133.67 96.52) (width 0.25) (layer "F.Cu") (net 1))
 (segment (start 135.88 91.43) (end 135.89 91.44) (width 0.25) (layer "F.Cu") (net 2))
 (segment (start 142.32 86.36) (end 144.145 86.36) (width 0.25) (layer "F.Cu") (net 2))
 (segment (start 130.175 96.52) (end 132 96.52) (width 0.25) (layer "F.Cu") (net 2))
 (segment (start 134.7 91.43) (end 135.88 91.43) (width 0.25) (layer "F.Cu") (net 2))
 (segment (start 137.16 95.885) (end 138.43 97.155) (width 0.25) (layer "F.Cu") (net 2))
 (segment (start 135.89 91.44) (end 136.525 90.805) (width 0.25) (layer "F.Cu") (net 2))
 (segment (start 138.43 97.155) (end 139.9325 97.155) (width 0.25) (layer "F.Cu") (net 2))
 (via (at 130.175 96.52) (size 0.8) (drill 0.4) (layers "F.Cu" "B.Cu") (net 2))
 (via (at 137.16 95.885) (size 0.8) (drill 0.4) (layers "F.Cu" "B.Cu") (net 2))
 (via (at 136.525 90.805) (size 0.8) (drill 0.4) (layers "F.Cu" "B.Cu") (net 2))
 (via (at 144.145 86.36) (size 0.8) (drill 0.4) (layers "F.Cu" "B.Cu") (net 2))
 (segment (start 137.16 90.805) (end 138.43 92.075) (width 0.25) (layer "B.Cu") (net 2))
 (segment (start 135.255 90.17) (end 135.255 88.265) (width 0.25) (layer "B.Cu") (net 2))
 (segment (start 144.175 86.39) (end 147.345 86.39) (width 0.25) (layer "B.Cu") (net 2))
 (segment (start 144.145 86.36) (end 144.175 86.39) (width 0.25) (layer "B.Cu") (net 2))
 (segment (start 130.175 96.52) (end 136.525 96.52) (width 0.25) (layer "B.Cu") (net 2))
 (segment (start 135.89 90.805) (end 136.525 90.805) (width 0.25) (layer "B.Cu") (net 2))
 (segment (start 135.255 90.17) (end 135.89 90.805) (width 0.25) (layer "B.Cu") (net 2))
 (segment (start 135.255 88.265) (end 137.16 86.36) (width 0.25) (layer "B.Cu") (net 2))
 (segment (start 136.525 90.805) (end 137.16 90.805) (width 0.25) (layer "B.Cu") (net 2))
 (segment (start 138.43 94.615) (end 137.16 95.885) (width 0.25) (layer "B.Cu") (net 2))
 (segment (start 137.16 86.36) (end 144.145 86.36) (width 0.25) (layer "B.Cu") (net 2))
 (segment (start 138.43 92.075) (end 138.43 94.615) (width 0.25) (layer "B.Cu") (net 2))
 (segment (start 136.525 96.52) (end 137.16 95.885) (width 0.25) (layer "B.Cu") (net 2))
 (segment (start 132 92.79) (end 131.445 93.345) (width 0.25) (layer "F.Cu") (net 6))
 (segment (start 132 92.38) (end 132 92.79) (width 0.25) (layer "F.Cu") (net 6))
 (segment (start 131.445 93.345) (end 129.54 93.345) (width 0.25) (layer "F.Cu") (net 6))
 (via (at 129.54 93.345) (size 0.8) (drill 0.4) (layers "F.Cu" "B.Cu") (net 6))
 (segment (start 123.19 86.995) (end 123.825 86.36) (width 0.25) (layer "B.Cu") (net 6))
 (segment (start 123.825 86.36) (end 128.27 86.36) (width 0.25) (layer "B.Cu") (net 6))
 (segment (start 128.905 86.995) (end 128.905 92.71) (width 0.25) (layer "B.Cu") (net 6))
 (segment (start 124.86 89.93) (end 123.585 89.93) (width 0.25) (layer "B.Cu") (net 6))
 (segment (start 128.905 92.71) (end 129.54 93.345) (width 0.25) (layer "B.Cu") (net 6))
 (segment (start 123.585 89.93) (end 123.19 89.535) (width 0.25) (layer "B.Cu") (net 6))
 (segment (start 123.19 89.535) (end 123.19 86.995) (width 0.25) (layer "B.Cu") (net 6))
 (segment (start 128.27 86.36) (end 128.905 86.995) (width 0.25) (layer "B.Cu") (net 6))
 (segment (start 125.73 96.52) (end 128.27 96.52) (width 0.25) (layer "F.Cu") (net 9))
 (segment (start 128.27 96.52) (end 129.22 95.57) (width 0.25) (layer "F.Cu") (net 9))
 (segment (start 124.86 95.65) (end 125.73 96.52) (width 0.25) (layer "F.Cu") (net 9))
 (segment (start 124.86 94.68) (end 124.86 95.65) (width 0.25) (layer "F.Cu") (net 9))
 (segment (start 129.22 95.57) (end 132 95.57) (width 0.25) (layer "F.Cu") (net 9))
 (segment (start 127.36 92.68) (end 129.56 90.48) (width 0.25) (layer "F.Cu") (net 4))
 (segment (start 129.56 90.48) (end 132 90.48) (width 0.25) (layer "F.Cu") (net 4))
 (segment (start 137.16 85.09) (end 133.07 85.09) (width 0.25) (layer "F.Cu") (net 13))
 (segment (start 124.86 88.18) (end 126.68 86.36) (width 0.25) (layer "F.Cu") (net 13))
 (segment (start 133.07 85.09) (end 131.8 86.36) (width 0.25) (layer "F.Cu") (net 13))
 (segment (start 126.68 86.36) (end 131.8 86.36) (width 0.25) (layer "F.Cu") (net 13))
 (segment (start 137.48 85.41) (end 137.16 85.09) (width 0.25) (layer "F.Cu") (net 13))
 (segment (start 139.62 85.41) (end 137.48 85.41) (width 0.25) (layer "F.Cu") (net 13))
 (segment (start 128.59 97.47) (end 132 97.47) (width 0.25) (layer "F.Cu") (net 10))
 (segment (start 128.27 97.79) (end 128.59 97.47) (width 0.25) (layer "F.Cu") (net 10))
 (via (at 128.27 97.79) (size 0.8) (drill 0.4) (layers "F.Cu" "B.Cu") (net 10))
 (segment (start 127.36 96.88) (end 128.27 97.79) (width 0.25) (layer "B.Cu") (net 10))
 (segment (start 127.36 94.68) (end 127.36 96.88) (width 0.25) (layer "B.Cu") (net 10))
 (segment (start 136.61 88.18) (end 137.48 87.31) (width 0.25) (layer "F.Cu") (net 14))
 (segment (start 134.9 86.36) (end 134.9 87.985) (width 0.25) (layer "F.Cu") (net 14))
 (segment (start 134.705 88.18) (end 136.61 88.18) (width 0.25) (layer "F.Cu") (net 14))
 (segment (start 134.9 87.985) (end 134.705 88.18) (width 0.25) (layer "F.Cu") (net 14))
 (segment (start 127.36 88.18) (end 134.705 88.18) (width 0.25) (layer "F.Cu") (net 14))
 (segment (start 137.48 87.31) (end 139.62 87.31) (width 0.25) (layer "F.Cu") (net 14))
 (segment (start 145.1 85.41) (end 145.415 85.725) (width 0.25) (layer "F.Cu") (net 12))
 (segment (start 145.415 85.725) (end 145.415 88.265) (width 0.25) (layer "F.Cu") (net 12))
 (segment (start 146.08 88.93) (end 147.345 88.93) (width 0.25) (layer "F.Cu") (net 12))
 (segment (start 142.32 85.41) (end 145.1 85.41) (width 0.25) (layer "F.Cu") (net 12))
 (segment (start 145.415 88.265) (end 146.08 88.93) (width 0.25) (layer "F.Cu") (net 12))
 (segment (start 134.7 90.09) (end 135.255 89.535) (width 0.25) (layer "F.Cu") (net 3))
 (segment (start 135.255 89.535) (end 137.16 89.535) (width 0.25) (layer "F.Cu") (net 3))
 (segment (start 134.7 90.48) (end 134.7 90.09) (width 0.25) (layer "F.Cu") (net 3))
 (via (at 137.16 89.535) (size 0.8) (drill 0.4) (layers "F.Cu" "B.Cu") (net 3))
 (segment (start 137.16 89.535) (end 137.795 90.17) (width 0.25) (layer "B.Cu") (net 3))
 (segment (start 146.045 90.17) (end 147.345 91.47) (width 0.25) (layer "B.Cu") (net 3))
 (segment (start 137.795 90.17) (end 146.045 90.17) (width 0.25) (layer "B.Cu") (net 3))
 (segment (start 137.16 97.79) (end 136.84 97.47) (width 0.25) (layer "F.Cu") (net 7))
 (segment (start 136.84 97.47) (end 134.7 97.47) (width 0.25) (layer "F.Cu") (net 7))
 (via (at 137.16 97.79) (size 0.8) (drill 0.4) (layers "F.Cu" "B.Cu") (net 7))
 (segment (start 143.565 97.79) (end 143.51 97.79) (width 0.25) (layer "B.Cu") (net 7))
 (segment (start 147.345 94.01) (end 143.565 97.79) (width 0.25) (layer "B.Cu") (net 7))
 (segment (start 143.51 97.79) (end 137.16 97.79) (width 0.25) (layer "B.Cu") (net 7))
 (segment (start 135.89 94.615) (end 139.97 94.615) (width 0.25) (layer "F.Cu") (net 8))
 (segment (start 134.935 95.57) (end 135.89 94.615) (width 0.25) (layer "F.Cu") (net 8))
 (segment (start 134.7 95.57) (end 134.935 95.57) (width 0.25) (layer "F.Cu") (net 8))
 (segment (start 137.7055 92.075) (end 137.16 92.6205) (width 0.25) (layer "F.Cu") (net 5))
 (segment (start 130.2645 91.457369) (end 131.972631 91.457369) (width 0.25) (layer "F.Cu") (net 5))
 (segment (start 131.972631 91.457369) (end 132 91.43) (width 0.25) (layer "F.Cu") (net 5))
 (segment (start 139.97 92.075) (end 137.7055 92.075) (width 0.25) (layer "F.Cu") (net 5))
 (via (at 137.16 92.6205) (size 0.8) (drill 0.4) (layers "F.Cu" "B.Cu") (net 5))
 (via (at 130.2645 91.457369) (size 0.8) (drill 0.4) (layers "F.Cu" "B.Cu") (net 5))
 (segment (start 130.2645 91.5295) (end 130.2645 91.457369) (width 0.25) (layer "B.Cu") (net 5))
 (segment (start 137.0705 92.71) (end 131.445 92.71) (width 0.25) (layer "B.Cu") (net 5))
 (segment (start 137.16 92.6205) (end 137.0705 92.71) (width 0.25) (layer "B.Cu") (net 5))
 (segment (start 131.445 92.71) (end 130.2645 91.5295) (width 0.25) (layer "B.Cu") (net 5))
 (segment (start 139.62 86.36) (end 140.65 86.36) (width 0.25) (layer "F.Cu") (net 11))
 (segment (start 140.65 86.36) (end 140.97 86.68) (width 0.25) (layer "F.Cu") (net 11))
 (segment (start 140.97 88.535) (end 139.97 89.535) (width 0.25) (layer "F.Cu") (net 11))
 (segment (start 140.97 86.68) (end 140.97 88.535) (width 0.25) (layer "F.Cu") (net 11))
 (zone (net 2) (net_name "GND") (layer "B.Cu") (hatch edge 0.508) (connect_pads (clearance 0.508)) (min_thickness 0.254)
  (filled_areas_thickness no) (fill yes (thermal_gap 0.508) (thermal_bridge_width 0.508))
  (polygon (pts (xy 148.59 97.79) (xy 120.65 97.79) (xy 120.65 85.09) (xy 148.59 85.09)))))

